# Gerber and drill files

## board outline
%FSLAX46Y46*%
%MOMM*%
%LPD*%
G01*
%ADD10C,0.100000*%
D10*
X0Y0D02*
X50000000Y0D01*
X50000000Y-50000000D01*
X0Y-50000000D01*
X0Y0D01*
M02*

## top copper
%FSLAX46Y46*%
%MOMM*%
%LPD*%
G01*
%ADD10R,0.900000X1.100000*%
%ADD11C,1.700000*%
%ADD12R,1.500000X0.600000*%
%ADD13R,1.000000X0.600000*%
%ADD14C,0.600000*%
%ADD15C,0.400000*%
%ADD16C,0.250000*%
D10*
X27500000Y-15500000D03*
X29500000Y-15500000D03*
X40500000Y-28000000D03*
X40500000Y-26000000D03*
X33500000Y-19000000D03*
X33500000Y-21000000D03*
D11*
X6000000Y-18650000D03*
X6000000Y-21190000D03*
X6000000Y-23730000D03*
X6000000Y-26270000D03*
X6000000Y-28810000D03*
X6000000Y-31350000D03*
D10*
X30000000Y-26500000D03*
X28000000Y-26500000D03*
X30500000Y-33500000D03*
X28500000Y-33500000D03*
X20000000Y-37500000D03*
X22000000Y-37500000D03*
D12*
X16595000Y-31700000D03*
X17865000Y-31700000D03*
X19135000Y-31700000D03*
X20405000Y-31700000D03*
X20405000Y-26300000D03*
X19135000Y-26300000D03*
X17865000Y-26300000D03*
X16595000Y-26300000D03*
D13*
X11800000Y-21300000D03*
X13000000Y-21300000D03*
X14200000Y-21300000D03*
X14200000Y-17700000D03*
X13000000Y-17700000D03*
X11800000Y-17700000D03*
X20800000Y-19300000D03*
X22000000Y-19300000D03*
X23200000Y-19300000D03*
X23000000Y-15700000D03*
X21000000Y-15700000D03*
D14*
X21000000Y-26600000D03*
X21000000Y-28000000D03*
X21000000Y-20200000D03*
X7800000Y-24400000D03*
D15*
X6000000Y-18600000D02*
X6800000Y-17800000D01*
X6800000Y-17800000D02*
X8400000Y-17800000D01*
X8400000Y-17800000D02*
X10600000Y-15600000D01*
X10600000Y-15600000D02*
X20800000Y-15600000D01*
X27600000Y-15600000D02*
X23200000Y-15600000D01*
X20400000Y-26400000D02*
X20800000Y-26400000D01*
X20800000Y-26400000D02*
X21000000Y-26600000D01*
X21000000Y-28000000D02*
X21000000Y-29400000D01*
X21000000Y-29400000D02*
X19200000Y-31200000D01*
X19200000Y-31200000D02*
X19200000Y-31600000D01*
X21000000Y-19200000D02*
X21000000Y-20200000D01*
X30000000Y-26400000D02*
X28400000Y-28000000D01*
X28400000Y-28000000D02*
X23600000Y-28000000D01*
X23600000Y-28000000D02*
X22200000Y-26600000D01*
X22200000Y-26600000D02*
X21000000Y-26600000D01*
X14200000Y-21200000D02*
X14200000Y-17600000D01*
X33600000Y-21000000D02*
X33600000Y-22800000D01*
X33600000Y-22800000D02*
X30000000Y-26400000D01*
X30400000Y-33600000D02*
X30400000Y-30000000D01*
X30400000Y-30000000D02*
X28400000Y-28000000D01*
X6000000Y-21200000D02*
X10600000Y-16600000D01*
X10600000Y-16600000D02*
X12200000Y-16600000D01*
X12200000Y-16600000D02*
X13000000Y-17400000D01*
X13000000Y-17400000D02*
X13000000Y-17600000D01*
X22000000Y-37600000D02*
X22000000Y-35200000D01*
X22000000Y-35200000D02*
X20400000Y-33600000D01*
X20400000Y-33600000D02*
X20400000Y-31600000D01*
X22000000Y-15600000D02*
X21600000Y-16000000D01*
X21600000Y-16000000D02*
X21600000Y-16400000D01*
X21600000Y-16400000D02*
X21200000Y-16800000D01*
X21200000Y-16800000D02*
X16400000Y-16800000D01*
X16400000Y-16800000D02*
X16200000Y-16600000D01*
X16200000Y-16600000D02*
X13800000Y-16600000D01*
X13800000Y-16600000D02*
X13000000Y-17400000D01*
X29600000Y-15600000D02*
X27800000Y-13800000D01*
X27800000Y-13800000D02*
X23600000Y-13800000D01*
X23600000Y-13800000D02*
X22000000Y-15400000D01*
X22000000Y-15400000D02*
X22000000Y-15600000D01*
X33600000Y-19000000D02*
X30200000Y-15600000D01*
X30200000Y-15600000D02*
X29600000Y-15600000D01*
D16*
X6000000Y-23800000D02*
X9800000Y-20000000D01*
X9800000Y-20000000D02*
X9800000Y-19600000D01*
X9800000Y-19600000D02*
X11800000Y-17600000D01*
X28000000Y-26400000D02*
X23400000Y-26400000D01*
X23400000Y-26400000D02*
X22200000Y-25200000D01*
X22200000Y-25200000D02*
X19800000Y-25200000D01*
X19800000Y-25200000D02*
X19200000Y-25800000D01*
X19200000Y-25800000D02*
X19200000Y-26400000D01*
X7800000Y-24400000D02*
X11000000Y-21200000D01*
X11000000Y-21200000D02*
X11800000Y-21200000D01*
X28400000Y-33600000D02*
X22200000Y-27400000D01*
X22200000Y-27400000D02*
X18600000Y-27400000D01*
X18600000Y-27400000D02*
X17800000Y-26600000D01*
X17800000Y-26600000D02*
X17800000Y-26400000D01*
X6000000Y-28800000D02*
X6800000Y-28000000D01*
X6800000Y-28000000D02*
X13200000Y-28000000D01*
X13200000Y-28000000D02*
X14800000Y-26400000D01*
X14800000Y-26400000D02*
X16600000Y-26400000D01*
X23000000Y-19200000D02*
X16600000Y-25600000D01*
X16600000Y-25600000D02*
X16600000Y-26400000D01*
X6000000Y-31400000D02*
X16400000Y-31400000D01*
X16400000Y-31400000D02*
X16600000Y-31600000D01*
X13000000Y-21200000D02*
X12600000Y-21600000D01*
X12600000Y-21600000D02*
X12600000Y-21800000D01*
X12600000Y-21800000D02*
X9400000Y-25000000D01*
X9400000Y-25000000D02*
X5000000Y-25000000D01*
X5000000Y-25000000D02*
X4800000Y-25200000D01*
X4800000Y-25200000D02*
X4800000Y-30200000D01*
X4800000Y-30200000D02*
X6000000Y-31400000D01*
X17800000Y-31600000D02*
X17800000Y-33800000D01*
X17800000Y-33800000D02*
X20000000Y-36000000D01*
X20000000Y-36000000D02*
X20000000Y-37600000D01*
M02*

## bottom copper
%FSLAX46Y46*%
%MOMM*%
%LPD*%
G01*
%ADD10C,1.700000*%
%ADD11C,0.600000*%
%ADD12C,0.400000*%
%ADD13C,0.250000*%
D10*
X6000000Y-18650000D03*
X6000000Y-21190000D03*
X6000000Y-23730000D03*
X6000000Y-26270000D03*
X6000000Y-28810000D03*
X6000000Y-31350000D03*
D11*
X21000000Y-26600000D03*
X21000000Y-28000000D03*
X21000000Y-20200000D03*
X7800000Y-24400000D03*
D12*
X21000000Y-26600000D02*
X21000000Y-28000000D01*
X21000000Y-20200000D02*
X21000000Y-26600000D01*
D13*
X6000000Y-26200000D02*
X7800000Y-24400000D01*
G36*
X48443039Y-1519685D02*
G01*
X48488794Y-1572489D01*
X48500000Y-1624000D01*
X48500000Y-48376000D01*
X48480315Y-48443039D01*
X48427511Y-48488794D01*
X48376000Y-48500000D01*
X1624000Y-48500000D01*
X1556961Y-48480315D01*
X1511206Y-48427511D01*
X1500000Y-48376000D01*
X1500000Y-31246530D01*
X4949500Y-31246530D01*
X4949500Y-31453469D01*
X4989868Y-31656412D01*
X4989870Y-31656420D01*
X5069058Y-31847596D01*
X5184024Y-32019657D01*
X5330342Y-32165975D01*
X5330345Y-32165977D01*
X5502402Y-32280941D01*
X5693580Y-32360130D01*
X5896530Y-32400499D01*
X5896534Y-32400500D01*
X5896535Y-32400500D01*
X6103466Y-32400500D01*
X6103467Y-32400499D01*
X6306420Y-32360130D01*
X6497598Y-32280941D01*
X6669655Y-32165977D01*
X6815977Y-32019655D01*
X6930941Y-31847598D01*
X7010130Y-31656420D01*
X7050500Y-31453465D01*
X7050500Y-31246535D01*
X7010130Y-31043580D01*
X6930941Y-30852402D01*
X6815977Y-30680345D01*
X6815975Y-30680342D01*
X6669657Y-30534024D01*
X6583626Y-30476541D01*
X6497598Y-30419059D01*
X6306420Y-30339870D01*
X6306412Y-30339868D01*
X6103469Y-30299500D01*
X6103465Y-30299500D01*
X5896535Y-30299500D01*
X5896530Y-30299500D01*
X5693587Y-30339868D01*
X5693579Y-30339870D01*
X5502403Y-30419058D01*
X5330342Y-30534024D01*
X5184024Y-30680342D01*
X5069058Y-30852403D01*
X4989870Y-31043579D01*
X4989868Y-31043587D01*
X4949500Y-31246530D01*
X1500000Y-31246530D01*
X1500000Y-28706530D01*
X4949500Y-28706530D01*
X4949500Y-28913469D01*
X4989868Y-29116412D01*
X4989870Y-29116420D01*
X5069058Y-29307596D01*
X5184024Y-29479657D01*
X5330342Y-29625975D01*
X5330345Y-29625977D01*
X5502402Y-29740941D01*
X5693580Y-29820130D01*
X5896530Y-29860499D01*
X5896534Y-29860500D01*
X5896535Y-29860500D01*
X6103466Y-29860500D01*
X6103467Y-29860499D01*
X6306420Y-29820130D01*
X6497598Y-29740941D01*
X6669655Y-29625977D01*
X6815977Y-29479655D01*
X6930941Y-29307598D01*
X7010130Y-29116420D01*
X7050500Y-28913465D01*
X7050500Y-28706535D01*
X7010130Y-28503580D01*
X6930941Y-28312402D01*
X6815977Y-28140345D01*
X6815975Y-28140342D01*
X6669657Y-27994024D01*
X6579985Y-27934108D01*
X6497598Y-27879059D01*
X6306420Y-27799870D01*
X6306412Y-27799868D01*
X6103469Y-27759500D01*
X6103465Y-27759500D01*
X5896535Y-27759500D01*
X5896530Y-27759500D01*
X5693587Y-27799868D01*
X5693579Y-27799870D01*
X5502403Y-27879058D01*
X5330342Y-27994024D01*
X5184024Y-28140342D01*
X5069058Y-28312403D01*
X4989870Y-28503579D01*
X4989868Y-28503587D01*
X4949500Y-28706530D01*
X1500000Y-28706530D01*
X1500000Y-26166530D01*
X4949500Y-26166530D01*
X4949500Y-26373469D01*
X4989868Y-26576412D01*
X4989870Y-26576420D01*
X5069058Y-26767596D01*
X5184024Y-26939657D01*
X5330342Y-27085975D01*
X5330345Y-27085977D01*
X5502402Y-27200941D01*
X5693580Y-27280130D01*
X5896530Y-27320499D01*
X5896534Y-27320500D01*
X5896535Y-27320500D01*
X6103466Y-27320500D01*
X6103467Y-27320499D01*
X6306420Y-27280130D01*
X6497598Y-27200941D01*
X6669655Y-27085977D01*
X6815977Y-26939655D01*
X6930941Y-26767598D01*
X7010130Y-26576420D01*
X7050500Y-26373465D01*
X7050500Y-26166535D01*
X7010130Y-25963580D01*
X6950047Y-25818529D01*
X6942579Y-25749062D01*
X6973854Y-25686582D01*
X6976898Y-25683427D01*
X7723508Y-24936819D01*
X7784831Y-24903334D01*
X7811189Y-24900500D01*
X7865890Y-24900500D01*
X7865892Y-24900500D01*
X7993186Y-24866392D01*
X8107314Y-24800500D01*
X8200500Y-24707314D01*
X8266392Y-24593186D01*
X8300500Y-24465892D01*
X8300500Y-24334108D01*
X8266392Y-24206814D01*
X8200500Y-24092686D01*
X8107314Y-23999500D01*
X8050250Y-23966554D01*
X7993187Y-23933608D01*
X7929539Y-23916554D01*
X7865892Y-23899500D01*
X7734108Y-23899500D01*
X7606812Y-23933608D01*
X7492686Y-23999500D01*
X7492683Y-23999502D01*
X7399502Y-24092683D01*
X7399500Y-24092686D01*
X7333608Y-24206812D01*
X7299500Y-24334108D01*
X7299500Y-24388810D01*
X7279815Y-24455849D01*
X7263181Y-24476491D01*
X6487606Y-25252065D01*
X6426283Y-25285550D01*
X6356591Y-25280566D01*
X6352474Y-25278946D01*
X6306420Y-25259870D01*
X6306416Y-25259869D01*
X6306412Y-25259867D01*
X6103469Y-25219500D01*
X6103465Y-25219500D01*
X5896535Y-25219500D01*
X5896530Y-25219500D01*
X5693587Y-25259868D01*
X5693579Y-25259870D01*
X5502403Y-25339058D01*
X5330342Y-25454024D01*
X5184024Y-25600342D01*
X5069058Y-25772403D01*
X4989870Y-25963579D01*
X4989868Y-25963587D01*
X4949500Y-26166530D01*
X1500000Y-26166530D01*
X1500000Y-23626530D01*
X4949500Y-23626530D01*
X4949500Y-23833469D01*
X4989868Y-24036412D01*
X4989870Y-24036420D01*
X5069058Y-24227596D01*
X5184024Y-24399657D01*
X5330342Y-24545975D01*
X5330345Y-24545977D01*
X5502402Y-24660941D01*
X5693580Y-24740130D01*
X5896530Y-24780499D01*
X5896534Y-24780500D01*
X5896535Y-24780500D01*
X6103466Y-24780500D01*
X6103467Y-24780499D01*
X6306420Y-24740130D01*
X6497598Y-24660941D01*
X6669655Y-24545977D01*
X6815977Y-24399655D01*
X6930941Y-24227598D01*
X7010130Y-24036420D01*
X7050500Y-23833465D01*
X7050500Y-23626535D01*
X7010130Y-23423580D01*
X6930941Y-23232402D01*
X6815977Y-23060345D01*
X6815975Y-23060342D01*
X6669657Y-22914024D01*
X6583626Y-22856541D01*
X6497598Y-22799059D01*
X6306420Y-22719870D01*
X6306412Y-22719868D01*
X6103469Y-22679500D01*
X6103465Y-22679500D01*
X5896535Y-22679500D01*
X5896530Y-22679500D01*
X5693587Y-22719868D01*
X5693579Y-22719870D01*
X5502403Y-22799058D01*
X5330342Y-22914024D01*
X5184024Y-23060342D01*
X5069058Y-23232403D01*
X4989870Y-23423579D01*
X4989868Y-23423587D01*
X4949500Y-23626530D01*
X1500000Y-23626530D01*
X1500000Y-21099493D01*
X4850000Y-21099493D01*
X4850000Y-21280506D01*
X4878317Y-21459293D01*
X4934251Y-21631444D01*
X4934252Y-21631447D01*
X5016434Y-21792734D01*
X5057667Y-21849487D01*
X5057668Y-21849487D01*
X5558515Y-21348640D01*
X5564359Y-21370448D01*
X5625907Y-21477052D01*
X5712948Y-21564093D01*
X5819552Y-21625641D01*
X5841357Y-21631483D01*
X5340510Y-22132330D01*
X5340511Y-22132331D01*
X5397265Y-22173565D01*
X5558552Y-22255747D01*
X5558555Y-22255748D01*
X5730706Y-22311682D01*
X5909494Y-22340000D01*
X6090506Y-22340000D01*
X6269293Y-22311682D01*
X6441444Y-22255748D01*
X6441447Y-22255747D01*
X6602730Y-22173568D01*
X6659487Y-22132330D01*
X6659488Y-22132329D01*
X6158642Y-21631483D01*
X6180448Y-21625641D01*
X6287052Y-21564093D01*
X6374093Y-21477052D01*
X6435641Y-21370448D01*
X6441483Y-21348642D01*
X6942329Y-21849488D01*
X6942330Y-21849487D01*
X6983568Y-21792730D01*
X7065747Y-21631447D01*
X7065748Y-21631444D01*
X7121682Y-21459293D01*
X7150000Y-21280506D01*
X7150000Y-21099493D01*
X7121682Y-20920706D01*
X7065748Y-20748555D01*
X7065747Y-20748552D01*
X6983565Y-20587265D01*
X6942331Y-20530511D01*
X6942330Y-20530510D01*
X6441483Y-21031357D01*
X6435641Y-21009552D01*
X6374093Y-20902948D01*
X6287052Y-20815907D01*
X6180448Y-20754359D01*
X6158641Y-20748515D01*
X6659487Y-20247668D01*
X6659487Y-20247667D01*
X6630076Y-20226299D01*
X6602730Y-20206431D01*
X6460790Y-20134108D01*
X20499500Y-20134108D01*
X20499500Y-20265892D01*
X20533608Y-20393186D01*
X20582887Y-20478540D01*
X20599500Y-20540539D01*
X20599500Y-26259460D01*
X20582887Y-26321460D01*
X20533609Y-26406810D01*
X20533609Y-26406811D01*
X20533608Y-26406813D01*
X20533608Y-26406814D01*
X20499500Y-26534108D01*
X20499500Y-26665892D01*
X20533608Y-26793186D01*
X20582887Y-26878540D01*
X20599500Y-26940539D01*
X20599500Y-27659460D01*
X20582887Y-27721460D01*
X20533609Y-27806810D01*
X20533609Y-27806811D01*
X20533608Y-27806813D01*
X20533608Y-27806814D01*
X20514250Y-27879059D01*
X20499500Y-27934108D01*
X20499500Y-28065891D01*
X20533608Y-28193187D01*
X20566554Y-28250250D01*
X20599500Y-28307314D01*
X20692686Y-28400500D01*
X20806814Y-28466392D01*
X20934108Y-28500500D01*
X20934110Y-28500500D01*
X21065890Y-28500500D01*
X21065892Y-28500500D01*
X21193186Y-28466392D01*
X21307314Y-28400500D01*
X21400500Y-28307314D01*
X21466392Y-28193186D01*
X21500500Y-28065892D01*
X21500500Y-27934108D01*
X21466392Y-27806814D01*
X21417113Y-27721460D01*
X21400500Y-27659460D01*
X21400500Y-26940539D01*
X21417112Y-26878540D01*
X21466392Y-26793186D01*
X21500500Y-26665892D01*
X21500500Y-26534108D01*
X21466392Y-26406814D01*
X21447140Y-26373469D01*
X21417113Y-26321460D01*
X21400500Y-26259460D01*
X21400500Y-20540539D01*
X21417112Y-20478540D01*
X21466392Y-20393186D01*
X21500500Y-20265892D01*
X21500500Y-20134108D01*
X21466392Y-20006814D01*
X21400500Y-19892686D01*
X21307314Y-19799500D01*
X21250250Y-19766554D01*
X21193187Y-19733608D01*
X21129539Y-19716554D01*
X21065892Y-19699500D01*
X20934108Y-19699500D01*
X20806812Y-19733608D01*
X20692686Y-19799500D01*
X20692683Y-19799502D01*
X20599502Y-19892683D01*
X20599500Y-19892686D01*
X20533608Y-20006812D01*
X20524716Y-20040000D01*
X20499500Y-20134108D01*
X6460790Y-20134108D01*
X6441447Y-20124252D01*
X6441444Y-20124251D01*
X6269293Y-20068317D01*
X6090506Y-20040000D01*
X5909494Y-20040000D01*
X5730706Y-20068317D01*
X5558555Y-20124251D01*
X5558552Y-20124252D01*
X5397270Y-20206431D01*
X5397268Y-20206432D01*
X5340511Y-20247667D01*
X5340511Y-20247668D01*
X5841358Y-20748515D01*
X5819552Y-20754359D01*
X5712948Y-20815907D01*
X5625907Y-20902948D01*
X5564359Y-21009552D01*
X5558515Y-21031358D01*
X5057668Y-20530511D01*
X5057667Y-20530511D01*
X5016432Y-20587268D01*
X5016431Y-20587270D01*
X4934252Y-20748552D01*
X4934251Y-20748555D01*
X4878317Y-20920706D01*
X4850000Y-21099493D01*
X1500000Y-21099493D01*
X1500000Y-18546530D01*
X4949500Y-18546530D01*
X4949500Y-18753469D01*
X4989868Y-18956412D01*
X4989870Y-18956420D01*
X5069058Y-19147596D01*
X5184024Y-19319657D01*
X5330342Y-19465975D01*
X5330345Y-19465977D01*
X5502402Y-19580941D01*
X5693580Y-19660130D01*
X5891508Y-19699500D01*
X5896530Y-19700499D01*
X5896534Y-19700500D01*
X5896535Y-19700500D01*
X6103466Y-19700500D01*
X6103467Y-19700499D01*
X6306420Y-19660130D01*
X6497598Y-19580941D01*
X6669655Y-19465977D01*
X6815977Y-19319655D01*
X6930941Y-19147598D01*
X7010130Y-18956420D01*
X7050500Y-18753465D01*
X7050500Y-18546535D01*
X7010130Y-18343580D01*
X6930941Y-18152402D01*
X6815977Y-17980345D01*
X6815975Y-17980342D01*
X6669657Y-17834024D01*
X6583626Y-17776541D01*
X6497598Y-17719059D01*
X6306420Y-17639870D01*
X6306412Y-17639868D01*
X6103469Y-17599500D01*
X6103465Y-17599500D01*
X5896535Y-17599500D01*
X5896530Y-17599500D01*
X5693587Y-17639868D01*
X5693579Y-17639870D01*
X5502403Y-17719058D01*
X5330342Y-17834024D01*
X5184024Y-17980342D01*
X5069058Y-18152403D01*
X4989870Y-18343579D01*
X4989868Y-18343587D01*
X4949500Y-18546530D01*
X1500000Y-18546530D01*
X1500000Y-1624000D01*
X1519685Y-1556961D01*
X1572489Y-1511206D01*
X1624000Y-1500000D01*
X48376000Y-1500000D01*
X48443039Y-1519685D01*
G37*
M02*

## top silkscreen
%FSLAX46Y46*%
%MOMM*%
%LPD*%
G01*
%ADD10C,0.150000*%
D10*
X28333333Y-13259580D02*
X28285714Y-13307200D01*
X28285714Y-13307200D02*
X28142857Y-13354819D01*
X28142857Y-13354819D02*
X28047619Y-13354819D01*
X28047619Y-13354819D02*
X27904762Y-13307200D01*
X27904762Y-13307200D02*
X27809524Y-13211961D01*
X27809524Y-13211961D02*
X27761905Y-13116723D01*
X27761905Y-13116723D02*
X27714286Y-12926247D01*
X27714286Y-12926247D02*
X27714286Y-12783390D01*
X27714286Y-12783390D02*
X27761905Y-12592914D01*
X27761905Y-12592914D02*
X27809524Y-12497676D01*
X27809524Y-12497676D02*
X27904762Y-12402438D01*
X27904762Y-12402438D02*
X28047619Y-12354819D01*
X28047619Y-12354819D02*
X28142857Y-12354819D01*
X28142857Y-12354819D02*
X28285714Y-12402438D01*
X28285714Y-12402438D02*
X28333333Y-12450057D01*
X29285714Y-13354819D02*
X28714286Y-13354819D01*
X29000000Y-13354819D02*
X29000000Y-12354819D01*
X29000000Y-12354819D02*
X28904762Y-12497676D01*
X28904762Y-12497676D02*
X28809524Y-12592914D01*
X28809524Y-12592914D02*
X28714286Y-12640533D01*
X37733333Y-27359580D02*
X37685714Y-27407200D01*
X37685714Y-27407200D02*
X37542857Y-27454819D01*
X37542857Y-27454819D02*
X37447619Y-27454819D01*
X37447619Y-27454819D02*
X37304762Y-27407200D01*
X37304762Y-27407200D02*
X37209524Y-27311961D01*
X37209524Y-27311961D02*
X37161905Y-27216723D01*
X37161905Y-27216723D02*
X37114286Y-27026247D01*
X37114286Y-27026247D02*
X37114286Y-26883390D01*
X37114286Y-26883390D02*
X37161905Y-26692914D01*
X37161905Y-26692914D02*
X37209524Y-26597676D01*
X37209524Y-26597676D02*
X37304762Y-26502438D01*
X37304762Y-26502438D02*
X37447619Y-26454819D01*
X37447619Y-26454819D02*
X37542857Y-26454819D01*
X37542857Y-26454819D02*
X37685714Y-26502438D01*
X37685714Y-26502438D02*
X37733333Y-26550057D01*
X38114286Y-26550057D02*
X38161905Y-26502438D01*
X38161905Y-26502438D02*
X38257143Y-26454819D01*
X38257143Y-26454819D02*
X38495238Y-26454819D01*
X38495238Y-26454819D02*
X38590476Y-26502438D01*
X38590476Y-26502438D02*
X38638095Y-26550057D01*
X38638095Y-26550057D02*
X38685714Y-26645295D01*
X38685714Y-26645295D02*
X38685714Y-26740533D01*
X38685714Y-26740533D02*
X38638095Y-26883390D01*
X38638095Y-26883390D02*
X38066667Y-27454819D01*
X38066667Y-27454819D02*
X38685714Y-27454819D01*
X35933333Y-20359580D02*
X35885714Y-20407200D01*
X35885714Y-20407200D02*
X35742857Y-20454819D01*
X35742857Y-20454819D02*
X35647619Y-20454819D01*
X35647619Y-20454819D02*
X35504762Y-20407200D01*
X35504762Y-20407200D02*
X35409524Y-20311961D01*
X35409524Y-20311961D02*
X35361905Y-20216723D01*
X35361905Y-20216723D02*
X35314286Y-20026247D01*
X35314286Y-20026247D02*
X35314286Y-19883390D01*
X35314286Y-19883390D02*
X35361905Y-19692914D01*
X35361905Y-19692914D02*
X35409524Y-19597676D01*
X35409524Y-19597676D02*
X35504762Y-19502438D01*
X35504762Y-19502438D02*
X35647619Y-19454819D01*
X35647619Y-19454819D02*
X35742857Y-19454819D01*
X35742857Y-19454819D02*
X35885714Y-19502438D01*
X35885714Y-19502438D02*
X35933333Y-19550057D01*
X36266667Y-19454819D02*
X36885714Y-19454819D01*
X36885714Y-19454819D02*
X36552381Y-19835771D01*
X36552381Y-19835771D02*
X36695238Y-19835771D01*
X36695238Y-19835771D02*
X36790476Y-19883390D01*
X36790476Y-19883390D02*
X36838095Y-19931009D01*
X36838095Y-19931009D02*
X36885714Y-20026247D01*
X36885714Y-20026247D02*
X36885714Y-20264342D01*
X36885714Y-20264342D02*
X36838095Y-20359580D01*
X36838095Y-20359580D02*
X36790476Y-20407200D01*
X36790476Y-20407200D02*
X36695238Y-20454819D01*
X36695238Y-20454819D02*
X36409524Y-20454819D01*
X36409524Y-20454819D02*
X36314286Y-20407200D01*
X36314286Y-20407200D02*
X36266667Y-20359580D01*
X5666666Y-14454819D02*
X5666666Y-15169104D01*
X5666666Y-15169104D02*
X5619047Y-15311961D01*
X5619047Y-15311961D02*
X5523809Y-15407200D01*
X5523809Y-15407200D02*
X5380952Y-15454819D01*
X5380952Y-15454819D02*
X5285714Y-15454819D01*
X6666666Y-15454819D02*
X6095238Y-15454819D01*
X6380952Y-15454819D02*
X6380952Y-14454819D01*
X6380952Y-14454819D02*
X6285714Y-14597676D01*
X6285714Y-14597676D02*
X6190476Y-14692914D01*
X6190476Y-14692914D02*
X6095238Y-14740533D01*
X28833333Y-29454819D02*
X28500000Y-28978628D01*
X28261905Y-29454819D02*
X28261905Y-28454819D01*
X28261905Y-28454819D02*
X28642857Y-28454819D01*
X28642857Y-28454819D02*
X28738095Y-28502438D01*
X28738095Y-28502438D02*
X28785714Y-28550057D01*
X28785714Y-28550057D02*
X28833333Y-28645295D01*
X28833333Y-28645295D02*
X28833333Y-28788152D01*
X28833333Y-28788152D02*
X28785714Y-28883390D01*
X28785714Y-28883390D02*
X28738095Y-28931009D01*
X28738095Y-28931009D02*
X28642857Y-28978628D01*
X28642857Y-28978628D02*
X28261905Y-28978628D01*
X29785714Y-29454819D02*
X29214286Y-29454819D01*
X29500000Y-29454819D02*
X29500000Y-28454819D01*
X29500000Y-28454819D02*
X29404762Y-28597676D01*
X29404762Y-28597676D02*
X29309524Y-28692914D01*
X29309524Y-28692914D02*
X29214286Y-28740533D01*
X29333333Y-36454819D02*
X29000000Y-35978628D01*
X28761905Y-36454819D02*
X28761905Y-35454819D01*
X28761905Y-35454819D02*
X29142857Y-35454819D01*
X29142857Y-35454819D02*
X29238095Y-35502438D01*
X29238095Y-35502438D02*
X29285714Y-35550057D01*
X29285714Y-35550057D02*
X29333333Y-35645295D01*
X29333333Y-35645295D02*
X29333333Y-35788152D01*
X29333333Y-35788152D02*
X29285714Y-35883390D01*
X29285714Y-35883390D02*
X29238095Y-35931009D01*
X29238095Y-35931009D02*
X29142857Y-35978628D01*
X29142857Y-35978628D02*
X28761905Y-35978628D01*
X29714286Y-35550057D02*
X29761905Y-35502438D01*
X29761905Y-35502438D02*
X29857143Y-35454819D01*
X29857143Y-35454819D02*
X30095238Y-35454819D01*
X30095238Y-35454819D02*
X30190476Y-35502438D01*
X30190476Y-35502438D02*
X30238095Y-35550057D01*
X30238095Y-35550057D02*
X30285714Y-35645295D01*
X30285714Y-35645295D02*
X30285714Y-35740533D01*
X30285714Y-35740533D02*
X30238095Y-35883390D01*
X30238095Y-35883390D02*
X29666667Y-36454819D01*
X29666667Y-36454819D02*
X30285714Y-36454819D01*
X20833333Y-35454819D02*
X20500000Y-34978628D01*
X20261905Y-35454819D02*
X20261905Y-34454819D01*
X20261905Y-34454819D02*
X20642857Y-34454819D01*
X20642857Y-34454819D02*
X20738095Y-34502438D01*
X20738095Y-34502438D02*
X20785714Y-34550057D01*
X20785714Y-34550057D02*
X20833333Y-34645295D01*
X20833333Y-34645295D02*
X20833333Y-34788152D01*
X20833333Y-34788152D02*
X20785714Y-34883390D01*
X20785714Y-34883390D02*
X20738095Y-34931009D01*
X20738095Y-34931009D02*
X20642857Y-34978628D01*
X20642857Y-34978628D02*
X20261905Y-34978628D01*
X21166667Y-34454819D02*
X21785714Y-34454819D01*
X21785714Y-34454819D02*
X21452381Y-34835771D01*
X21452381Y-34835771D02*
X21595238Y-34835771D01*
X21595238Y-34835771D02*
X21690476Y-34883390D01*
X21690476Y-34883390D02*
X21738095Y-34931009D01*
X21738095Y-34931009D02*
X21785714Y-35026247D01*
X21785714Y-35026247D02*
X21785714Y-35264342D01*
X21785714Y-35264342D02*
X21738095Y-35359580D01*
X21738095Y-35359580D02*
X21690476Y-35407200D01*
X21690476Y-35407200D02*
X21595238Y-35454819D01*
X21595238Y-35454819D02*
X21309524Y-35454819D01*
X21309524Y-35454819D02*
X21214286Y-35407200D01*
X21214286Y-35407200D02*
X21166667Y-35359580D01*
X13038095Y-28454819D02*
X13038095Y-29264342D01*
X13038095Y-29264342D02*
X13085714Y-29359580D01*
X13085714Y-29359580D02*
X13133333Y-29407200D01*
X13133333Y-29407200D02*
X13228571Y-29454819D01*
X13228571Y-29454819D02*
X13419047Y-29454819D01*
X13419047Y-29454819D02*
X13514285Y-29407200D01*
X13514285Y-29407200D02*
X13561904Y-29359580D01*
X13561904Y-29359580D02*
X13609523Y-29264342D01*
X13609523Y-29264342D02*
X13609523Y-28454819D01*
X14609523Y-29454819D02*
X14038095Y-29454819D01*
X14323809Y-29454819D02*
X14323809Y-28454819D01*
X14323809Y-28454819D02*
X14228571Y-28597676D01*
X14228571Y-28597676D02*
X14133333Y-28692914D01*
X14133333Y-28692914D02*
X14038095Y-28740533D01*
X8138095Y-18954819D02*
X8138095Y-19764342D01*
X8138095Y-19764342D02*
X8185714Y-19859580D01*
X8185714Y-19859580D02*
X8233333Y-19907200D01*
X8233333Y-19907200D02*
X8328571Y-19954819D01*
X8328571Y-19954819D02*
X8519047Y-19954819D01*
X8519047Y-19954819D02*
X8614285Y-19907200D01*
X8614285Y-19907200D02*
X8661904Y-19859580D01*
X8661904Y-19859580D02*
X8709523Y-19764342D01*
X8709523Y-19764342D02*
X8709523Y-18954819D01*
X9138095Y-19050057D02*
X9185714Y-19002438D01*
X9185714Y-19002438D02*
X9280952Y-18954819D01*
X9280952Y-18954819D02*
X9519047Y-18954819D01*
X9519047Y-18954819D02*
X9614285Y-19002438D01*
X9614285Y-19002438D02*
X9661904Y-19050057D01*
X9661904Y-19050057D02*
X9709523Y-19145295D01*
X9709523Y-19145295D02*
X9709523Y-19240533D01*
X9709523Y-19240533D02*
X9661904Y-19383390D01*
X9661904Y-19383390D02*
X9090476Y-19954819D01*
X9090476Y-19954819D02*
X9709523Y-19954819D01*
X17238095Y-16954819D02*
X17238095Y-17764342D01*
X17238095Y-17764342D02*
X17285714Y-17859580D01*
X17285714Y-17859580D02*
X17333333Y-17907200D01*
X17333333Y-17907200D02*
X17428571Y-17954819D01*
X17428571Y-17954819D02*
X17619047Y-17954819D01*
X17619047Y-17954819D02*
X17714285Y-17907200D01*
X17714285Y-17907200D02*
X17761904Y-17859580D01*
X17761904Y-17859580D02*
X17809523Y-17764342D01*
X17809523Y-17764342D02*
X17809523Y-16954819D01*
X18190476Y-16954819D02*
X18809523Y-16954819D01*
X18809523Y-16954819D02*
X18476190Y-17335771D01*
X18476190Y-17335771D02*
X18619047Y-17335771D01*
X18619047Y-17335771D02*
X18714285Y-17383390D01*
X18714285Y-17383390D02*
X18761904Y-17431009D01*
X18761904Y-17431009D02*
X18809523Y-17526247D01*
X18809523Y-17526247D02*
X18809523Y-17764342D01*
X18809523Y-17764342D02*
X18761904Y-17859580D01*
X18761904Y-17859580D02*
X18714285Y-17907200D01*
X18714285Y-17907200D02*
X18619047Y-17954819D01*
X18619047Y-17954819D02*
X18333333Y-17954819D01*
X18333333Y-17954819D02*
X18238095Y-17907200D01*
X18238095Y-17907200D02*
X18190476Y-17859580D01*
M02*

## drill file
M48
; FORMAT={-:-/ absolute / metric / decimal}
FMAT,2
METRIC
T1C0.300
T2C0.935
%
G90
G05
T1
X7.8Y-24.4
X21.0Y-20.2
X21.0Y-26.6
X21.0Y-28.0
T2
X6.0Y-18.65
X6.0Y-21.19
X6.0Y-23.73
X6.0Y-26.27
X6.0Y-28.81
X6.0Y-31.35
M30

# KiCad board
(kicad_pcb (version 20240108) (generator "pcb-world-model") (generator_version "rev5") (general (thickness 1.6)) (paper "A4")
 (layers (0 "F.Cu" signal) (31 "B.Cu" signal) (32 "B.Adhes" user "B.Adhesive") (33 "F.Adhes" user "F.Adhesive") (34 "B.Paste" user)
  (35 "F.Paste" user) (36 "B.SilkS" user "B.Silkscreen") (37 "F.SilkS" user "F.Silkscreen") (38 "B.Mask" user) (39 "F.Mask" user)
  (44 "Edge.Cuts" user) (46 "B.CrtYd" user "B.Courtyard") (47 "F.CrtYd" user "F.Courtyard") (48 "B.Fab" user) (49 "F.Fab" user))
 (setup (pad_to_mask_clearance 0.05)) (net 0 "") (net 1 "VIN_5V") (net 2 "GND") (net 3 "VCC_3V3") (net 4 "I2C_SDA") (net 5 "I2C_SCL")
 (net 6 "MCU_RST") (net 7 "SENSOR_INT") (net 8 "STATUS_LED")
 (gr_rect (start 0.0 0.0) (end 50.0000 50.0000) (stroke (width 0.1) (type default)) (fill none) (layer "Edge.Cuts"))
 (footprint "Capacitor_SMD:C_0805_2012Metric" (layer "F.Cu") (at 28.5000 15.5000 0)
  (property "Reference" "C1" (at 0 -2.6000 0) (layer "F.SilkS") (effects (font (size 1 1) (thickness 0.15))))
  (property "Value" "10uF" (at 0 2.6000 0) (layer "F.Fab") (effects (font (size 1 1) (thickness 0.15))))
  (pad "1" smd rect (at -1.0000 0.0000) (size 0.9000 1.1000) (layers "F.Cu" "F.Paste" "F.Mask") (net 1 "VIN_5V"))
  (pad "2" smd rect (at 1.0000 0.0000) (size 0.9000 1.1000) (layers "F.Cu" "F.Paste" "F.Mask") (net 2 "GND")))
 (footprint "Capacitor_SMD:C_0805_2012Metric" (layer "F.Cu") (at 40.5000 27.0000 90)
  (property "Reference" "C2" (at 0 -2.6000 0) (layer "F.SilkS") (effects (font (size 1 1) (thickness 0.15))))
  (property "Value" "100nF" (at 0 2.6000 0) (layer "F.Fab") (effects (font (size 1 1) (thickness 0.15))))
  (pad "1" smd rect (at -1.0000 0.0000) (size 0.9000 1.1000) (layers "F.Cu" "F.Paste" "F.Mask") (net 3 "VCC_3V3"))
  (pad "2" smd rect (at 1.0000 0.0000) (size 0.9000 1.1000) (layers "F.Cu" "F.Paste" "F.Mask") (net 2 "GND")))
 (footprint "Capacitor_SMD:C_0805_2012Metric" (layer "F.Cu") (at 33.5000 20.0000 270)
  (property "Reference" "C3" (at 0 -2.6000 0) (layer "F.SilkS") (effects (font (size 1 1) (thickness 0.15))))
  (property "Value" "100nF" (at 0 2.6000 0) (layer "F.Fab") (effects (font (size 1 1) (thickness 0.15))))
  (pad "1" smd rect (at -1.0000 0.0000) (size 0.9000 1.1000) (layers "F.Cu" "F.Paste" "F.Mask") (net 3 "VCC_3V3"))
  (pad "2" smd rect (at 1.0000 0.0000) (size 0.9000 1.1000) (layers "F.Cu" "F.Paste" "F.Mask") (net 2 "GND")))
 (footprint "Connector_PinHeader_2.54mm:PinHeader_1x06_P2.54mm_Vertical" (layer "F.Cu") (at 6.0000 25.0000 0) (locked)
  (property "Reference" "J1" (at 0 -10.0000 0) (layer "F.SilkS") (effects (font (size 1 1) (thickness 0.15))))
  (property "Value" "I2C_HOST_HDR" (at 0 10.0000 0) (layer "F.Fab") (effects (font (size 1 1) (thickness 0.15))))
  (pad "1" thru_hole circle (at 0.0000 -6.3500) (size 1.7000 1.7000) (drill 0.9350) (layers "*.Cu" "*.Mask") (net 1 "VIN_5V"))
  (pad "2" thru_hole circle (at 0.0000 -3.8100) (size 1.7000 1.7000) (drill 0.9350) (layers "*.Cu" "*.Mask") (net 2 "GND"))
  (pad "3" thru_hole circle (at 0.0000 -1.2700) (size 1.7000 1.7000) (drill 0.9350) (layers "*.Cu" "*.Mask") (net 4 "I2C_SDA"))
  (pad "4" thru_hole circle (at 0.0000 1.2700) (size 1.7000 1.7000) (drill 0.9350) (layers "*.Cu" "*.Mask") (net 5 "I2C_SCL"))
  (pad "5" thru_hole circle (at 0.0000 3.8100) (size 1.7000 1.7000) (drill 0.9350) (layers "*.Cu" "*.Mask") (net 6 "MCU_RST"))
  (pad "6" thru_hole circle (at 0.0000 6.3500) (size 1.7000 1.7000) (drill 0.9350) (layers "*.Cu" "*.Mask") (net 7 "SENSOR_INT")))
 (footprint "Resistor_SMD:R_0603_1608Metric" (layer "F.Cu") (at 29.0000 26.5000 180)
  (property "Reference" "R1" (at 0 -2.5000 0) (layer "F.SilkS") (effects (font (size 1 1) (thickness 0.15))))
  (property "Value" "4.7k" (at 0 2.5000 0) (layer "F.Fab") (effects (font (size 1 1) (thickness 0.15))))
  (pad "1" smd rect (at -1.0000 0.0000) (size 0.9000 1.1000) (layers "F.Cu" "F.Paste" "F.Mask") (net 3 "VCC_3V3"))
  (pad "2" smd rect (at 1.0000 0.0000) (size 0.9000 1.1000) (layers "F.Cu" "F.Paste" "F.Mask") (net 4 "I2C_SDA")))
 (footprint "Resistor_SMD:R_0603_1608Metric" (layer "F.Cu") (at 29.5000 33.5000 180)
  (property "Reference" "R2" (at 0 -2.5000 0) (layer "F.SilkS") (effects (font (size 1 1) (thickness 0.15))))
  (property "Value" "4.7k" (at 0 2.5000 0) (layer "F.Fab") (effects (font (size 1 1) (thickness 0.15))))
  (pad "1" smd rect (at -1.0000 0.0000) (size 0.9000 1.1000) (layers "F.Cu" "F.Paste" "F.Mask") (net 3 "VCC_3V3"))
  (pad "2" smd rect (at 1.0000 0.0000) (size 0.9000 1.1000) (layers "F.Cu" "F.Paste" "F.Mask") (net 5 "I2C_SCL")))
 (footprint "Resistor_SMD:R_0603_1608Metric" (layer "F.Cu") (at 21.0000 37.5000 0)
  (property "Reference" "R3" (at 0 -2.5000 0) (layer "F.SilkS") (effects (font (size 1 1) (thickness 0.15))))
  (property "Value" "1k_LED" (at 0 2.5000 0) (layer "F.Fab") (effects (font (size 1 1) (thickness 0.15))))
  (pad "1" smd rect (at -1.0000 0.0000) (size 0.9000 1.1000) (layers "F.Cu" "F.Paste" "F.Mask") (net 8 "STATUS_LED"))
  (pad "2" smd rect (at 1.0000 0.0000) (size 0.9000 1.1000) (layers "F.Cu" "F.Paste" "F.Mask") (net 2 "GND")))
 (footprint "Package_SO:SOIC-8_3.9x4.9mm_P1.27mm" (layer "F.Cu") (at 18.5000 29.0000 90)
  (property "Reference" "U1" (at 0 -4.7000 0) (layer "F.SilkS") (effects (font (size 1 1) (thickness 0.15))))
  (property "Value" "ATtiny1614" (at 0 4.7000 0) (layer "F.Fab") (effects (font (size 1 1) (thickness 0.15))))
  (pad "1" smd rect (at -2.7000 -1.9050) (size 1.5000 0.6000) (layers "F.Cu" "F.Paste" "F.Mask") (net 3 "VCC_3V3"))
  (pad "2" smd rect (at -2.7000 -0.6350) (size 1.5000 0.6000) (layers "F.Cu" "F.Paste" "F.Mask") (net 4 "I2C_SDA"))
  (pad "3" smd rect (at -2.7000 0.6350) (size 1.5000 0.6000) (layers "F.Cu" "F.Paste" "F.Mask") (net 5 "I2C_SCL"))
  (pad "4" smd rect (at -2.7000 1.9050) (size 1.5000 0.6000) (layers "F.Cu" "F.Paste" "F.Mask") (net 6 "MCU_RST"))
  (pad "5" smd rect (at 2.7000 1.9050) (size 1.5000 0.6000) (layers "F.Cu" "F.Paste" "F.Mask") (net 7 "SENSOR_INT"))
  (pad "6" smd rect (at 2.7000 0.6350) (size 1.5000 0.6000) (layers "F.Cu" "F.Paste" "F.Mask") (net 8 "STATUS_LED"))
  (pad "7" smd rect (at 2.7000 -0.6350) (size 1.5000 0.6000) (layers "F.Cu" "F.Paste" "F.Mask") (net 3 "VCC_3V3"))
  (pad "8" smd rect (at 2.7000 -1.9050) (size 1.5000 0.6000) (layers "F.Cu" "F.Paste" "F.Mask") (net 2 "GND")))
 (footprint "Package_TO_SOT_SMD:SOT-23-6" (layer "F.Cu") (at 13.0000 19.5000 90)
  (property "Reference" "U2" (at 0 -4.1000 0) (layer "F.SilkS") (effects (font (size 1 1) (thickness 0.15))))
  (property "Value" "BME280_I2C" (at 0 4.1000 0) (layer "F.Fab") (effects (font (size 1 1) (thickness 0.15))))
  (pad "1" smd rect (at -1.8000 -1.2000) (size 1.0000 0.6000) (layers "F.Cu" "F.Paste" "F.Mask") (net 3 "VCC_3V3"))
  (pad "2" smd rect (at -1.8000 0.0000) (size 1.0000 0.6000) (layers "F.Cu" "F.Paste" "F.Mask") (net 2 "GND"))
  (pad "3" smd rect (at -1.8000 1.2000) (size 1.0000 0.6000) (layers "F.Cu" "F.Paste" "F.Mask") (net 4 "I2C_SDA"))
  (pad "4" smd rect (at 1.8000 1.2000) (size 1.0000 0.6000) (layers "F.Cu" "F.Paste" "F.Mask") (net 5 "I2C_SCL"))
  (pad "5" smd rect (at 1.8000 0.0000) (size 1.0000 0.6000) (layers "F.Cu" "F.Paste" "F.Mask") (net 7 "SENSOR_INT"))
  (pad "6" smd rect (at 1.8000 -1.2000) (size 1.0000 0.6000) (layers "F.Cu" "F.Paste" "F.Mask") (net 3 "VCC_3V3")))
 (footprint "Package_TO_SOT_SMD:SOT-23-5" (layer "F.Cu") (at 22.0000 17.5000 90)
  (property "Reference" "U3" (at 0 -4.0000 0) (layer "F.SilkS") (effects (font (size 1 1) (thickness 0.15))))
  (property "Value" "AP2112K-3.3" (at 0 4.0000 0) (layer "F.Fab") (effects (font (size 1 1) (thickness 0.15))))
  (pad "1" smd rect (at -1.8000 -1.2000) (size 1.0000 0.6000) (layers "F.Cu" "F.Paste" "F.Mask") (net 1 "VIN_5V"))
  (pad "2" smd rect (at -1.8000 0.0000) (size 1.0000 0.6000) (layers "F.Cu" "F.Paste" "F.Mask") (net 2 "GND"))
  (pad "3" smd rect (at -1.8000 1.2000) (size 1.0000 0.6000) (layers "F.Cu" "F.Paste" "F.Mask") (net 1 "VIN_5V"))
  (pad "4" smd rect (at 1.8000 1.0000) (size 1.0000 0.6000) (layers "F.Cu" "F.Paste" "F.Mask") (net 3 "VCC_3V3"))
  (pad "5" smd rect (at 1.8000 -1.0000) (size 1.0000 0.6000) (layers "F.Cu" "F.Paste" "F.Mask") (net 6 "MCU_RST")))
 (segment (start 6.0000 18.6000) (end 6.8000 17.8000) (width 0.4000) (layer "F.Cu") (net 1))
 (segment (start 6.8000 17.8000) (end 8.4000 17.8000) (width 0.4000) (layer "F.Cu") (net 1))
 (segment (start 8.4000 17.8000) (end 10.6000 15.6000) (width 0.4000) (layer "F.Cu") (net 1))
 (segment (start 10.6000 15.6000) (end 20.8000 15.6000) (width 0.4000) (layer "F.Cu") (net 1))
 (segment (start 27.6000 15.6000) (end 23.2000 15.6000) (width 0.4000) (layer "F.Cu") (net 1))
 (segment (start 20.4000 26.4000) (end 20.8000 26.4000) (width 0.4000) (layer "F.Cu") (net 3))
 (segment (start 20.8000 26.4000) (end 21.0000 26.6000) (width 0.4000) (layer "F.Cu") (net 3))
 (segment (start 21.0000 26.6000) (end 21.0000 28.0000) (width 0.4000) (layer "B.Cu") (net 3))
 (segment (start 21.0000 28.0000) (end 21.0000 29.4000) (width 0.4000) (layer "F.Cu") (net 3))
 (segment (start 21.0000 29.4000) (end 19.2000 31.2000) (width 0.4000) (layer "F.Cu") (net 3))
 (segment (start 19.2000 31.2000) (end 19.2000 31.6000) (width 0.4000) (layer "F.Cu") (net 3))
 (segment (start 21.0000 19.2000) (end 21.0000 20.2000) (width 0.4000) (layer "F.Cu") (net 3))
 (segment (start 21.0000 20.2000) (end 21.0000 26.6000) (width 0.4000) (layer "B.Cu") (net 3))
 (segment (start 30.0000 26.4000) (end 28.4000 28.0000) (width 0.4000) (layer "F.Cu") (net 3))
 (segment (start 28.4000 28.0000) (end 23.6000 28.0000) (width 0.4000) (layer "F.Cu") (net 3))
 (segment (start 23.6000 28.0000) (end 22.2000 26.6000) (width 0.4000) (layer "F.Cu") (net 3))
 (segment (start 22.2000 26.6000) (end 21.0000 26.6000) (width 0.4000) (layer "F.Cu") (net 3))
 (segment (start 14.2000 21.2000) (end 14.2000 17.6000) (width 0.4000) (layer "F.Cu") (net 3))
 (segment (start 33.6000 21.0000) (end 33.6000 22.8000) (width 0.4000) (layer "F.Cu") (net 3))
 (segment (start 33.6000 22.8000) (end 30.0000 26.4000) (width 0.4000) (layer "F.Cu") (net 3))
 (segment (start 30.4000 33.6000) (end 30.4000 30.0000) (width 0.4000) (layer "F.Cu") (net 3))
 (segment (start 30.4000 30.0000) (end 28.4000 28.0000) (width 0.4000) (layer "F.Cu") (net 3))
 (segment (start 6.0000 21.2000) (end 10.6000 16.6000) (width 0.4000) (layer "F.Cu") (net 2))
 (segment (start 10.6000 16.6000) (end 12.2000 16.6000) (width 0.4000) (layer "F.Cu") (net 2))
 (segment (start 12.2000 16.6000) (end 13.0000 17.4000) (width 0.4000) (layer "F.Cu") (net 2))
 (segment (start 13.0000 17.4000) (end 13.0000 17.6000) (width 0.4000) (layer "F.Cu") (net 2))
 (segment (start 22.0000 37.6000) (end 22.0000 35.2000) (width 0.4000) (layer "F.Cu") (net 2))
 (segment (start 22.0000 35.2000) (end 20.4000 33.6000) (width 0.4000) (layer "F.Cu") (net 2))
 (segment (start 20.4000 33.6000) (end 20.4000 31.6000) (width 0.4000) (layer "F.Cu") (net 2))
 (segment (start 22.0000 15.6000) (end 21.6000 16.0000) (width 0.4000) (layer "F.Cu") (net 2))
 (segment (start 21.6000 16.0000) (end 21.6000 16.4000) (width 0.4000) (layer "F.Cu") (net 2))
 (segment (start 21.6000 16.4000) (end 21.2000 16.8000) (width 0.4000) (layer "F.Cu") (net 2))
 (segment (start 21.2000 16.8000) (end 16.4000 16.8000) (width 0.4000) (layer "F.Cu") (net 2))
 (segment (start 16.4000 16.8000) (end 16.2000 16.6000) (width 0.4000) (layer "F.Cu") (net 2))
 (segment (start 16.2000 16.6000) (end 13.8000 16.6000) (width 0.4000) (layer "F.Cu") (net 2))
 (segment (start 13.8000 16.6000) (end 13.0000 17.4000) (width 0.4000) (layer "F.Cu") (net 2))
 (segment (start 29.6000 15.6000) (end 27.8000 13.8000) (width 0.4000) (layer "F.Cu") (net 2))
 (segment (start 27.8000 13.8000) (end 23.6000 13.8000) (width 0.4000) (layer "F.Cu") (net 2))
 (segment (start 23.6000 13.8000) (end 22.0000 15.4000) (width 0.4000) (layer "F.Cu") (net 2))
 (segment (start 22.0000 15.4000) (end 22.0000 15.6000) (width 0.4000) (layer "F.Cu") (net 2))
 (segment (start 33.6000 19.0000) (end 30.2000 15.6000) (width 0.4000) (layer "F.Cu") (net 2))
 (segment (start 30.2000 15.6000) (end 29.6000 15.6000) (width 0.4000) (layer "F.Cu") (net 2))
 (segment (start 6.0000 23.8000) (end 9.8000 20.0000) (width 0.2500) (layer "F.Cu") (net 4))
 (segment (start 9.8000 20.0000) (end 9.8000 19.6000) (width 0.2500) (layer "F.Cu") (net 4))
 (segment (start 9.8000 19.6000) (end 11.8000 17.6000) (width 0.2500) (layer "F.Cu") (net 4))
 (segment (start 28.0000 26.4000) (end 23.4000 26.4000) (width 0.2500) (layer "F.Cu") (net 4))
 (segment (start 23.4000 26.4000) (end 22.2000 25.2000) (width 0.2500) (layer "F.Cu") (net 4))
 (segment (start 22.2000 25.2000) (end 19.8000 25.2000) (width 0.2500) (layer "F.Cu") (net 4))
 (segment (start 19.8000 25.2000) (end 19.2000 25.8000) (width 0.2500) (layer "F.Cu") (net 4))
 (segment (start 19.2000 25.8000) (end 19.2000 26.4000) (width 0.2500) (layer "F.Cu") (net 4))
 (segment (start 6.0000 26.2000) (end 7.8000 24.4000) (width 0.2500) (layer "B.Cu") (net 5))
 (segment (start 7.8000 24.4000) (end 11.0000 21.2000) (width 0.2500) (layer "F.Cu") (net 5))
 (segment (start 11.0000 21.2000) (end 11.8000 21.2000) (width 0.2500) (layer "F.Cu") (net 5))
 (segment (start 28.4000 33.6000) (end 22.2000 27.4000) (width 0.2500) (layer "F.Cu") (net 5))
 (segment (start 22.2000 27.4000) (end 18.6000 27.4000) (width 0.2500) (layer "F.Cu") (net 5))
 (segment (start 18.6000 27.4000) (end 17.8000 26.6000) (width 0.2500) (layer "F.Cu") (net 5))
 (segment (start 17.8000 26.6000) (end 17.8000 26.4000) (width 0.2500) (layer "F.Cu") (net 5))
 (segment (start 6.0000 28.8000) (end 6.8000 28.0000) (width 0.2500) (layer "F.Cu") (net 6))
 (segment (start 6.8000 28.0000) (end 13.2000 28.0000) (width 0.2500) (layer "F.Cu") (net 6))
 (segment (start 13.2000 28.0000) (end 14.8000 26.4000) (width 0.2500) (layer "F.Cu") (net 6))
 (segment (start 14.8000 26.4000) (end 16.6000 26.4000) (width 0.2500) (layer "F.Cu") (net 6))
 (segment (start 23.0000 19.2000) (end 16.6000 25.6000) (width 0.2500) (layer "F.Cu") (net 6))
 (segment (start 16.6000 25.6000) (end 16.6000 26.4000) (width 0.2500) (layer "F.Cu") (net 6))
 (segment (start 6.0000 31.4000) (end 16.4000 31.4000) (width 0.2500) (layer "F.Cu") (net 7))
 (segment (start 16.4000 31.4000) (end 16.6000 31.6000) (width 0.2500) (layer "F.Cu") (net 7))
 (segment (start 13.0000 21.2000) (end 12.6000 21.6000) (width 0.2500) (layer "F.Cu") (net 7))
 (segment (start 12.6000 21.6000) (end 12.6000 21.8000) (width 0.2500) (layer "F.Cu") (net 7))
 (segment (start 12.6000 21.8000) (end 9.4000 25.0000) (width 0.2500) (layer "F.Cu") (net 7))
 (segment (start 9.4000 25.0000) (end 5.0000 25.0000) (width 0.2500) (layer "F.Cu") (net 7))
 (segment (start 5.0000 25.0000) (end 4.8000 25.2000) (width 0.2500) (layer "F.Cu") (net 7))
 (segment (start 4.8000 25.2000) (end 4.8000 30.2000) (width 0.2500) (layer "F.Cu") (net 7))
 (segment (start 4.8000 30.2000) (end 6.0000 31.4000) (width 0.2500) (layer "F.Cu") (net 7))
 (segment (start 17.8000 31.6000) (end 17.8000 33.8000) (width 0.2500) (layer "F.Cu") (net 8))
 (segment (start 17.8000 33.8000) (end 20.0000 36.0000) (width 0.2500) (layer "F.Cu") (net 8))
 (segment (start 20.0000 36.0000) (end 20.0000 37.6000) (width 0.2500) (layer "F.Cu") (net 8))
 (via (at 21.0000 26.6000) (size 0.6000) (drill 0.3000) (layers "F.Cu" "B.Cu") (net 3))
 (via (at 21.0000 28.0000) (size 0.6000) (drill 0.3000) (layers "F.Cu" "B.Cu") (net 3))
 (via (at 21.0000 20.2000) (size 0.6000) (drill 0.3000) (layers "F.Cu" "B.Cu") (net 3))
 (via (at 7.8000 24.4000) (size 0.6000) (drill 0.3000) (layers "F.Cu" "B.Cu") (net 5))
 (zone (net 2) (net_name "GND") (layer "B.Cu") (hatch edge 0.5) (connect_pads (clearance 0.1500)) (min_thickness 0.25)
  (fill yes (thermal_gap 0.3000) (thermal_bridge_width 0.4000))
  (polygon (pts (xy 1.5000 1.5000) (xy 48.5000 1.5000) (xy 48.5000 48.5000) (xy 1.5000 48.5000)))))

